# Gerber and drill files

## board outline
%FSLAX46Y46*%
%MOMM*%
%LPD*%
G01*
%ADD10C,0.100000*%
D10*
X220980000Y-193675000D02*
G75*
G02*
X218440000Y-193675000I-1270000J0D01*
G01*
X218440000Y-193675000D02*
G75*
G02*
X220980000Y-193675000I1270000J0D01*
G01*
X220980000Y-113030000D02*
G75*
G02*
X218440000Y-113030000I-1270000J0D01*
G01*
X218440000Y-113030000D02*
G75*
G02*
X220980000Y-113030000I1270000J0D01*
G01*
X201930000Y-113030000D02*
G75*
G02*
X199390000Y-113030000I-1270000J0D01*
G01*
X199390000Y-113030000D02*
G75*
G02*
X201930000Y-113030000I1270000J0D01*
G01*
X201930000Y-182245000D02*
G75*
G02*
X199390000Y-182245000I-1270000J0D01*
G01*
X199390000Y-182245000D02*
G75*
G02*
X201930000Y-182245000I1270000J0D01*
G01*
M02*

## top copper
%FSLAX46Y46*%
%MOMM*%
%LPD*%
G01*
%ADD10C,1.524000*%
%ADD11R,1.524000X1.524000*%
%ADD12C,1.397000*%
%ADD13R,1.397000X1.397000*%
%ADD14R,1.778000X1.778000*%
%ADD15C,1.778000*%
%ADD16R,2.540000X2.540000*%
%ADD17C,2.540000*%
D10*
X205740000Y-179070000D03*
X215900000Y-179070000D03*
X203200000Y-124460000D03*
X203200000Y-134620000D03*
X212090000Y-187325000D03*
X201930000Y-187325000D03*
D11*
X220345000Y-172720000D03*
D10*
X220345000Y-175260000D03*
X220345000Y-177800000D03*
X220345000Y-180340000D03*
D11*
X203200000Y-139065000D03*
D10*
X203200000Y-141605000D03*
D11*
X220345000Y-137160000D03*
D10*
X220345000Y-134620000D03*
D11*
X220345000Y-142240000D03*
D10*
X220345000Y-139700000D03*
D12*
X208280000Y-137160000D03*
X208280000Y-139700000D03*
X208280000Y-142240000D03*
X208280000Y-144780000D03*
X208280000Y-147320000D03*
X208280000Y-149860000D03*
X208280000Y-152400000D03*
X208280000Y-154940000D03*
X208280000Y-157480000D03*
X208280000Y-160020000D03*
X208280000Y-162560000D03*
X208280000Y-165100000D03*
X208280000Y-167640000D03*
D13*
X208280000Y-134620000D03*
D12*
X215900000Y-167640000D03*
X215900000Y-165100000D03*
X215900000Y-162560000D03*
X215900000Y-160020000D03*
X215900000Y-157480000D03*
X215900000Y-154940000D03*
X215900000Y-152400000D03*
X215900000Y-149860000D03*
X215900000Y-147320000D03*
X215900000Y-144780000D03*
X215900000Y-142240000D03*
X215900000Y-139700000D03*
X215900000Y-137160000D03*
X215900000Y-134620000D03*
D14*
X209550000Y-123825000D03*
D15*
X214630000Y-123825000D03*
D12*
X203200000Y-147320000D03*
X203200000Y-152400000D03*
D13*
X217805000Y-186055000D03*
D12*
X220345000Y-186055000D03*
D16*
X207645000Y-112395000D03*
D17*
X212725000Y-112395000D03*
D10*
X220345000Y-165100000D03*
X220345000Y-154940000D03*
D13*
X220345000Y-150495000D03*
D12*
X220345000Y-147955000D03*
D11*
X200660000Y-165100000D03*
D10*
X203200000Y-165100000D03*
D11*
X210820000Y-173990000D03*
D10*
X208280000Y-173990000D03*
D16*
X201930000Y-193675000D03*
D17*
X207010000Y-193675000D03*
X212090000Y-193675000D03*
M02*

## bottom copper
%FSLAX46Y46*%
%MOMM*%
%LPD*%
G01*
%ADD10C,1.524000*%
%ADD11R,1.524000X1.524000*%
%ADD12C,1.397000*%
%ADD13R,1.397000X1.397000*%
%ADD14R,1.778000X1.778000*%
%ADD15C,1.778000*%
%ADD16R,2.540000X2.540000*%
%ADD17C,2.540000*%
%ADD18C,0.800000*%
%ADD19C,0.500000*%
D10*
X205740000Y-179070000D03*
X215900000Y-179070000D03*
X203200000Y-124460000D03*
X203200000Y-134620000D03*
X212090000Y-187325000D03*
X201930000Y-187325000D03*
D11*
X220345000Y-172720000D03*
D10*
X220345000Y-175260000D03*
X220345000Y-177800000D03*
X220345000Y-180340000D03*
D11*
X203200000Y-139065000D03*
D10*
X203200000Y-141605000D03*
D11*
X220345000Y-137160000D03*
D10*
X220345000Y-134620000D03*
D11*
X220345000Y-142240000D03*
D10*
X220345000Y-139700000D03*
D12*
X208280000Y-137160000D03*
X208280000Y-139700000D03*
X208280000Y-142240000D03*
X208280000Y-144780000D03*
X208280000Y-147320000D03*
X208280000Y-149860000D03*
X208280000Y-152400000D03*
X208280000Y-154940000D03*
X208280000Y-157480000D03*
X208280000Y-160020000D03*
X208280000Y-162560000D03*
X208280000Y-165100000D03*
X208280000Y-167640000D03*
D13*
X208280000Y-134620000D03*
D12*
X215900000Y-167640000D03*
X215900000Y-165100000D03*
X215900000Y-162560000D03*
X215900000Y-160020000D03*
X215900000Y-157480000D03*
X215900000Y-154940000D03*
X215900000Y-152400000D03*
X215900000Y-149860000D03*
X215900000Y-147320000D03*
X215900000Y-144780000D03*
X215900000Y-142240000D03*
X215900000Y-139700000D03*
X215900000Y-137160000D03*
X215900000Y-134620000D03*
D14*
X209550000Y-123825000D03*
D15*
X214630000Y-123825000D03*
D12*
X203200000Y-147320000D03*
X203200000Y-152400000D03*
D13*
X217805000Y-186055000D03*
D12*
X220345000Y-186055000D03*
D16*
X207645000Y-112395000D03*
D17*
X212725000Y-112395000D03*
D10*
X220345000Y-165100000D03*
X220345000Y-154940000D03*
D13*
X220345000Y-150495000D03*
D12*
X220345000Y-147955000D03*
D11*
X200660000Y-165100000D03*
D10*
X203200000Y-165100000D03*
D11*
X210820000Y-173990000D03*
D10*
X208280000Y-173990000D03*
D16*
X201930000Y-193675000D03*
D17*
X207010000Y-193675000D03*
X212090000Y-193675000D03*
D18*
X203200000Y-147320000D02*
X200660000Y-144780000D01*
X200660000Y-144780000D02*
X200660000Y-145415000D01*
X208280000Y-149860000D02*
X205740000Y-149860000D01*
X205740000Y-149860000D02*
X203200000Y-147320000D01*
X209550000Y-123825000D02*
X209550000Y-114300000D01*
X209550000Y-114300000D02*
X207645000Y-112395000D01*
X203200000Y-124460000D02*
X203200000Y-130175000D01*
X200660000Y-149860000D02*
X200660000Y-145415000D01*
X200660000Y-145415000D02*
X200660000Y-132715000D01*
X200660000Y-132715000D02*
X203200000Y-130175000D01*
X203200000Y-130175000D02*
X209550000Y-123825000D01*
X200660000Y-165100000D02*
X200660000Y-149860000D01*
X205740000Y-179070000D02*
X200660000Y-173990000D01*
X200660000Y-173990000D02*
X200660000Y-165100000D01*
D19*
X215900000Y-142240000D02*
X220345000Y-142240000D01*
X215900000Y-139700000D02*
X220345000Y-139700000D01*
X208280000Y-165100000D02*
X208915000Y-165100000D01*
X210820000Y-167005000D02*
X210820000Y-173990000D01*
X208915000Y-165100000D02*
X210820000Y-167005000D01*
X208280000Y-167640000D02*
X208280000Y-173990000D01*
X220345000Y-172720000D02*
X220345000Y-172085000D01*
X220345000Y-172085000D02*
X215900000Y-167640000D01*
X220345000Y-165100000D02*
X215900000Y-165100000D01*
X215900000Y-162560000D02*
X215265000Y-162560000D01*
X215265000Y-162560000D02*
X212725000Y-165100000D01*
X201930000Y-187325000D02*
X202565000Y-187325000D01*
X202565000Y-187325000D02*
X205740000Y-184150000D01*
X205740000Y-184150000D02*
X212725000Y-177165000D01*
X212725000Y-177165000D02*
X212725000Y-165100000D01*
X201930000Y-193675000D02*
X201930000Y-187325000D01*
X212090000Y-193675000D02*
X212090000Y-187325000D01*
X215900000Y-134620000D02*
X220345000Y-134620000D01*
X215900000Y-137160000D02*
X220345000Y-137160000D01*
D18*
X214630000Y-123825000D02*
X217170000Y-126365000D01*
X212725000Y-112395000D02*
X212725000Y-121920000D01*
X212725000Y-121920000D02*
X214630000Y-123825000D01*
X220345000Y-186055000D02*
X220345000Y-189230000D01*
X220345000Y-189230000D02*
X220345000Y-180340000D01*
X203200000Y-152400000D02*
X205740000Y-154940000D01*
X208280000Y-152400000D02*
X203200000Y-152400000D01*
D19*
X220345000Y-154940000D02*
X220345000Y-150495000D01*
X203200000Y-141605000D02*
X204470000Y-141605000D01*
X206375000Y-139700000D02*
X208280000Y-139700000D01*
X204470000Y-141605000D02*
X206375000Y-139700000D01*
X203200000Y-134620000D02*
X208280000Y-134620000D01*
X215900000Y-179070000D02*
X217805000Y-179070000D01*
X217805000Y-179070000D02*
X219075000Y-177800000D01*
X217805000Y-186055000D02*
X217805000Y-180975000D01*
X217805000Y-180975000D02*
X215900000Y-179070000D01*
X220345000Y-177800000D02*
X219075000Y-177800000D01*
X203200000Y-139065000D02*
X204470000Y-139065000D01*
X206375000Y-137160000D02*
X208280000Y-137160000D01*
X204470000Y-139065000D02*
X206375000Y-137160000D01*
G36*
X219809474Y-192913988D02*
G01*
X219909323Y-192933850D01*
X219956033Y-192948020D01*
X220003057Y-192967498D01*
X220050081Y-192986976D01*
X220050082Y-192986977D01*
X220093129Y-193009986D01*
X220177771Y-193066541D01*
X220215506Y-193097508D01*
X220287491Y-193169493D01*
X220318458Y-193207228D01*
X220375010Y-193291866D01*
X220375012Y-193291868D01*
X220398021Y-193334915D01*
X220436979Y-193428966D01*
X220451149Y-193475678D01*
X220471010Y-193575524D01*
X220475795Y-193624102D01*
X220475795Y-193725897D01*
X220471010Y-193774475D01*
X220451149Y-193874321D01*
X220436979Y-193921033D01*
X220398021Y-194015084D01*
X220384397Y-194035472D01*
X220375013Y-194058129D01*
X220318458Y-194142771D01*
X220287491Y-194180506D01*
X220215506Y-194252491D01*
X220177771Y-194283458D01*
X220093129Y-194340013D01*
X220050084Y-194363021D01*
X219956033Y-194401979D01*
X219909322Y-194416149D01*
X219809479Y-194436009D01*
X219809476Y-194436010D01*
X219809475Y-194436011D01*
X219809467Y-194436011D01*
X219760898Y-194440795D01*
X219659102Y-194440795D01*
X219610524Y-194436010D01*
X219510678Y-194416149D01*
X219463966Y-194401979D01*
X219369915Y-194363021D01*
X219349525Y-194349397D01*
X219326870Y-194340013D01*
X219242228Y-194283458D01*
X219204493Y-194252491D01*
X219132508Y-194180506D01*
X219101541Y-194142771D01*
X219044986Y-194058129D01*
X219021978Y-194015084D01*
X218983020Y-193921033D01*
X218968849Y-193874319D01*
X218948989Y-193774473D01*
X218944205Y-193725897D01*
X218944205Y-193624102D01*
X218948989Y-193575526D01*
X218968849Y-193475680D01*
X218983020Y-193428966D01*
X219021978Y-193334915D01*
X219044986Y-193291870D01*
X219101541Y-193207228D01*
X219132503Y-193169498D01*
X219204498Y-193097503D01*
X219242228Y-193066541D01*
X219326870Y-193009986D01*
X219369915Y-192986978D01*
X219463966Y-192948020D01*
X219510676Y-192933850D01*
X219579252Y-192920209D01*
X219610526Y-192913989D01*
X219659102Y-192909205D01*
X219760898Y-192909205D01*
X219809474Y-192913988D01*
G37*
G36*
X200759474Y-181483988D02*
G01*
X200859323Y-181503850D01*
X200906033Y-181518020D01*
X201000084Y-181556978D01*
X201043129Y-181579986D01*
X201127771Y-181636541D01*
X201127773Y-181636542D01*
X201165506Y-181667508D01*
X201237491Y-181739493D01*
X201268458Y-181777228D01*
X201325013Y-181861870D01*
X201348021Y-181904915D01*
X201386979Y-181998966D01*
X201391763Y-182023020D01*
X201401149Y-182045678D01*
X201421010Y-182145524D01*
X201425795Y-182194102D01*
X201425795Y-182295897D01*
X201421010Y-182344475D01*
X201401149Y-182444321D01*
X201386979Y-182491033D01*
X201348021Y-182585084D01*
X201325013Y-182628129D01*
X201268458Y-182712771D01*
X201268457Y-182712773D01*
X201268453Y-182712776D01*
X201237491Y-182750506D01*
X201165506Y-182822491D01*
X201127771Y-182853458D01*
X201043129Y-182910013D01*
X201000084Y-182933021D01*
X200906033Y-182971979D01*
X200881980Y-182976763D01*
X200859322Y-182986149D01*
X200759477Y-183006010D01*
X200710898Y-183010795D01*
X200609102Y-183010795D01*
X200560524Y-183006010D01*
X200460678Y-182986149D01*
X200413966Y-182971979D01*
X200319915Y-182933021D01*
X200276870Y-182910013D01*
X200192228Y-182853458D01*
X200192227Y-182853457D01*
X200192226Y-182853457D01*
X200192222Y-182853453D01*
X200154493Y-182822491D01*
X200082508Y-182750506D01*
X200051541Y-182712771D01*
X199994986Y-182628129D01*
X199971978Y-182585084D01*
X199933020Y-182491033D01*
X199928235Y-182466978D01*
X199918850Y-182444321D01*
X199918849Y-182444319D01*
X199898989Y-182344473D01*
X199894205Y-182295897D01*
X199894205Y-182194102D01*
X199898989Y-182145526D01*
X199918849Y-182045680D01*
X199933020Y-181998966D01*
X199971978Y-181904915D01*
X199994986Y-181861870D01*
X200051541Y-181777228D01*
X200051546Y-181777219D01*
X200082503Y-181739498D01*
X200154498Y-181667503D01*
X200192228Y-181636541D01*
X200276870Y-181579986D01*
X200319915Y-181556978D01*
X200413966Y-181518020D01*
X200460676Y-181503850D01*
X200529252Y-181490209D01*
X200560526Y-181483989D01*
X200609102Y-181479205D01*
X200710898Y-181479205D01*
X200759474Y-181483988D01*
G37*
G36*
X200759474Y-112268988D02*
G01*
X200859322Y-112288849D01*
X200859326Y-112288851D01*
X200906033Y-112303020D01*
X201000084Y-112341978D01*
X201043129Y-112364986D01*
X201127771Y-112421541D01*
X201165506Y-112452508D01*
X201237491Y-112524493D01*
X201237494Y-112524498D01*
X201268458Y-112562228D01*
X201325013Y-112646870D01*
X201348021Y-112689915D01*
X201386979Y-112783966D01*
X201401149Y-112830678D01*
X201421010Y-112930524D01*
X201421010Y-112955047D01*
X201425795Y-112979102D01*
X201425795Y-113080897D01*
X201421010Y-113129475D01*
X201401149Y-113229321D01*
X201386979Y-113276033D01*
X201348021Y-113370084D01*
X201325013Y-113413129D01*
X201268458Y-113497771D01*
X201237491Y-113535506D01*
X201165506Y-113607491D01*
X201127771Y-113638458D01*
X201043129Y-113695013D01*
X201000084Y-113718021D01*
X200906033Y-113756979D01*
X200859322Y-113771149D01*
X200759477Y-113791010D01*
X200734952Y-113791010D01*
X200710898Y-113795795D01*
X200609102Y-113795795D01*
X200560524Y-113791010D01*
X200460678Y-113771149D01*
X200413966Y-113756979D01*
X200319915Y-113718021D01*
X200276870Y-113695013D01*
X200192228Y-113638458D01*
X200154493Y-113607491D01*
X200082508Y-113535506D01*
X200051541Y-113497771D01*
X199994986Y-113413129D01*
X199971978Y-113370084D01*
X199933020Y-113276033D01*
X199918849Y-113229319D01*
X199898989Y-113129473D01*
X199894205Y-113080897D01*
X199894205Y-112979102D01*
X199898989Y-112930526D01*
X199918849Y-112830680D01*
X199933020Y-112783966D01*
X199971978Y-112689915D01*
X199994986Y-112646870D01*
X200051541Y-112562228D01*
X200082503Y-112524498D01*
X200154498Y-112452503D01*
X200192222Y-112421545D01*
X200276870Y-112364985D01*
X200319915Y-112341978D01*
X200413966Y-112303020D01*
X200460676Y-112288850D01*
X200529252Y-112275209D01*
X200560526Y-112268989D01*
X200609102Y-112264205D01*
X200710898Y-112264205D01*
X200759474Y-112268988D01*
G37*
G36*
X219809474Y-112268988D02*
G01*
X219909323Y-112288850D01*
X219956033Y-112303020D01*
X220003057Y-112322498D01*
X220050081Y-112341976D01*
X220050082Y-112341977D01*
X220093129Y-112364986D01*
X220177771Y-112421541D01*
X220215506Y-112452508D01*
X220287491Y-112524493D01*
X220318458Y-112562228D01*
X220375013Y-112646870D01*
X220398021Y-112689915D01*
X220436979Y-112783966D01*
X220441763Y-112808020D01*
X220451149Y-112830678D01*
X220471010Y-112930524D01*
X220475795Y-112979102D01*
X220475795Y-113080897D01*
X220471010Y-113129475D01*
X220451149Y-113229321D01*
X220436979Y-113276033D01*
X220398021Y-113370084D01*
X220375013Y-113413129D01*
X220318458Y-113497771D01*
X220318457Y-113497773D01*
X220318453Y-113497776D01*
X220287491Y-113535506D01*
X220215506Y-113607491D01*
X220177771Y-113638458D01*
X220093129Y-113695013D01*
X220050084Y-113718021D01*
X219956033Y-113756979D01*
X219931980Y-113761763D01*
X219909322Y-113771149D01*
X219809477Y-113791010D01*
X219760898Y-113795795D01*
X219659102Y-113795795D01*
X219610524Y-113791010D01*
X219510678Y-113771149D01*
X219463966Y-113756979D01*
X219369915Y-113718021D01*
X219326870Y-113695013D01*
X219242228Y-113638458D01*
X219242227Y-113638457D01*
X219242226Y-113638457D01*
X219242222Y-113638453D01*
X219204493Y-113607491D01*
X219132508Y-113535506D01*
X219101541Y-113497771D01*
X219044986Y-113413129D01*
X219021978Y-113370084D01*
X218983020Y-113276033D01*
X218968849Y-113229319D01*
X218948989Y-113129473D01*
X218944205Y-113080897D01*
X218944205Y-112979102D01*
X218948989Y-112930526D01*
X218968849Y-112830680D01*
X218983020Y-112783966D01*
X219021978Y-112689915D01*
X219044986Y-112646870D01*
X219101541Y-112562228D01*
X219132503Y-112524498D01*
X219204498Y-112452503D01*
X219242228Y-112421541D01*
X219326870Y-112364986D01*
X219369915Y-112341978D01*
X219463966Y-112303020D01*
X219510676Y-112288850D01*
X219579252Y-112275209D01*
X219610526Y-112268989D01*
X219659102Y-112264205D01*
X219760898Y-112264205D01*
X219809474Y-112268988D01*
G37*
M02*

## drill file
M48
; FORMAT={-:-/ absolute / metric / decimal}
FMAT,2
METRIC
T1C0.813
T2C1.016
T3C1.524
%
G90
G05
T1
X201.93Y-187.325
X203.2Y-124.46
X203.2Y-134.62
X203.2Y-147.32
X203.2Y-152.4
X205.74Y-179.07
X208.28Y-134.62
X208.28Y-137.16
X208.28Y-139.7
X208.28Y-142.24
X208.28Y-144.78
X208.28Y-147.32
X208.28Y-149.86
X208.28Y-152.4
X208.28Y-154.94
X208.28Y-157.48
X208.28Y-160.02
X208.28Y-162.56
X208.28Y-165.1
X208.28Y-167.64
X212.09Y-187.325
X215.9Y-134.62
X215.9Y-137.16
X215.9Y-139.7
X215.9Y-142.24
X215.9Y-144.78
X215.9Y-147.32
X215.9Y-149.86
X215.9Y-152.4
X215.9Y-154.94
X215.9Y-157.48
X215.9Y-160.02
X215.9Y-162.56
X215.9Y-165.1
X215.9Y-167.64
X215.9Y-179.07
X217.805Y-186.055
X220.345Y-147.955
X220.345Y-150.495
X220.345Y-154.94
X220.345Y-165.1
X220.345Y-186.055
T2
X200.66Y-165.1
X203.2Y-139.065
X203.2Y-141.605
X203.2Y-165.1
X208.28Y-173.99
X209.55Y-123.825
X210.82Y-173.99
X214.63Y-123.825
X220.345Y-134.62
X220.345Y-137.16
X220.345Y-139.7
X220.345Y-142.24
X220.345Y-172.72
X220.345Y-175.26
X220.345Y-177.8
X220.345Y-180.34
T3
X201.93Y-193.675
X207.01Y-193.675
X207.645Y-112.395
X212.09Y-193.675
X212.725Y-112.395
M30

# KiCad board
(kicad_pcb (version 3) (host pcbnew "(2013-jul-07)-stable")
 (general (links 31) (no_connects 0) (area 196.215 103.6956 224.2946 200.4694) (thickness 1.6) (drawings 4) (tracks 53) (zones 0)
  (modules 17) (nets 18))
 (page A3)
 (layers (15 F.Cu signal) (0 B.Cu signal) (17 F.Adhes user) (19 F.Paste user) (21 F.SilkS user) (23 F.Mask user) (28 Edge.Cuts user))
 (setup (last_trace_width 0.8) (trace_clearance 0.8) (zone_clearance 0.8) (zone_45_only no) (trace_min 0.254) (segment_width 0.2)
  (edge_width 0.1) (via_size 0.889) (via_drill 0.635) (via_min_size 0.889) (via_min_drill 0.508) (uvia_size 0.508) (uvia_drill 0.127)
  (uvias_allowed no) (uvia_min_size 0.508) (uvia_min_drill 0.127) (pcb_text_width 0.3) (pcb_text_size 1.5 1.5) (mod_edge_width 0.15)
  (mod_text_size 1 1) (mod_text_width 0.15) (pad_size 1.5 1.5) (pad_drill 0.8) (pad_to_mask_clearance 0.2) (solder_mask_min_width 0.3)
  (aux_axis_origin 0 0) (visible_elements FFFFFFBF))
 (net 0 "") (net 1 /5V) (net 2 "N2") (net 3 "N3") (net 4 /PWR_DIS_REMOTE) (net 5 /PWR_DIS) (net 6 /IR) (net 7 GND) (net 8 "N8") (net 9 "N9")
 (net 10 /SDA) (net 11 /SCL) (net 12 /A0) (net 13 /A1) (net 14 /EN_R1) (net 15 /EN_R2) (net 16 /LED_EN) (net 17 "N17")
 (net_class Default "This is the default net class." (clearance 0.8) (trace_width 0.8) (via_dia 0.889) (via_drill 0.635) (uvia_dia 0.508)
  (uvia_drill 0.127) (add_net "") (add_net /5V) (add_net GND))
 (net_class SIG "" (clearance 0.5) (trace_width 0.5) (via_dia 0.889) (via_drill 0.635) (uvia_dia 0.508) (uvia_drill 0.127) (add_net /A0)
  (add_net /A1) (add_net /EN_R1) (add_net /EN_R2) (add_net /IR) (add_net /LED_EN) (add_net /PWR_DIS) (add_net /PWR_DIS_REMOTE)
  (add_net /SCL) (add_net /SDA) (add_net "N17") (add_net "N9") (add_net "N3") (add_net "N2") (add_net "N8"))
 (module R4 (layer F.Cu) (at 210.82 179.07) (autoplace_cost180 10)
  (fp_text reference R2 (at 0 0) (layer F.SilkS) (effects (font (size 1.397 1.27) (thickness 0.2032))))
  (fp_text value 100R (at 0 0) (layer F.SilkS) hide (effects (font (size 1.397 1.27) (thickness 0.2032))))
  (pad 1 thru_hole circle (at -5.08 0) (size 1.524 1.524) (drill 0.8128) (layers *.Cu *.Mask F.SilkS) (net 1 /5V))
  (pad 2 thru_hole circle (at 5.08 0) (size 1.524 1.524) (drill 0.8128) (layers *.Cu *.Mask F.SilkS) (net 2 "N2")))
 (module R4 (layer F.Cu) (at 203.2 129.54 270) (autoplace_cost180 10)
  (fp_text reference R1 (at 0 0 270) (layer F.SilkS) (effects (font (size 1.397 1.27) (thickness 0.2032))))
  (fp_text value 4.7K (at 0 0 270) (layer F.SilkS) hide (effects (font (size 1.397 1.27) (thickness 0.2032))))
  (pad 1 thru_hole circle (at -5.08 0 270) (size 1.524 1.524) (drill 0.8128) (layers *.Cu *.Mask F.SilkS) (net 1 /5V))
  (pad 2 thru_hole circle (at 5.08 0 270) (size 1.524 1.524) (drill 0.8128) (layers *.Cu *.Mask F.SilkS) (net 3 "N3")))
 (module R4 (layer F.Cu) (at 207.01 187.325 180) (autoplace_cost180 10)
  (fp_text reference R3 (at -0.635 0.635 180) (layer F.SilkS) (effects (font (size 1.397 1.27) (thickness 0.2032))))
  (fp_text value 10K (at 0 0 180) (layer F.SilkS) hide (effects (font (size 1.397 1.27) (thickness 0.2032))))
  (pad 1 thru_hole circle (at -5.08 0 180) (size 1.524 1.524) (drill 0.8128) (layers *.Cu *.Mask F.SilkS) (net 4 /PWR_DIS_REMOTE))
  (pad 2 thru_hole circle (at 5.08 0 180) (size 1.524 1.524) (drill 0.8128) (layers *.Cu *.Mask F.SilkS) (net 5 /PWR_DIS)))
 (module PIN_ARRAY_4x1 (layer F.Cu) (at 220.345 176.53 270)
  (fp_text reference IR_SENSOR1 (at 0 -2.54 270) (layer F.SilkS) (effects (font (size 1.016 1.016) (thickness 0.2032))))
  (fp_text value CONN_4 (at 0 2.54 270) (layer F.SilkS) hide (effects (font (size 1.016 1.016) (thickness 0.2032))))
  (pad 1 thru_hole rect (at -3.81 0 270) (size 1.524 1.524) (drill 1.016) (layers *.Cu *.Mask F.SilkS) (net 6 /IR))
  (pad 2 thru_hole circle (at -1.27 0 270) (size 1.524 1.524) (drill 1.016) (layers *.Cu *.Mask F.SilkS))
  (pad 3 thru_hole circle (at 1.27 0 270) (size 1.524 1.524) (drill 1.016) (layers *.Cu *.Mask F.SilkS) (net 2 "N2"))
  (pad 4 thru_hole circle (at 3.81 0 270) (size 1.524 1.524) (drill 1.016) (layers *.Cu *.Mask F.SilkS) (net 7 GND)))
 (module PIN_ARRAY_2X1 (layer F.Cu) (at 203.2 140.335 270)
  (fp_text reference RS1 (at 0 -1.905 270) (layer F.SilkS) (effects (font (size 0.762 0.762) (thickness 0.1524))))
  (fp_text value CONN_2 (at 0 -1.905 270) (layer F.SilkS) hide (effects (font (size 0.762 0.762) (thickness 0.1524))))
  (pad 1 thru_hole rect (at -1.27 0 270) (size 1.524 1.524) (drill 1.016) (layers *.Cu *.Mask F.SilkS) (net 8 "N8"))
  (pad 2 thru_hole circle (at 1.27 0 270) (size 1.524 1.524) (drill 1.016) (layers *.Cu *.Mask F.SilkS) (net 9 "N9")))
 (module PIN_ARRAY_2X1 (layer F.Cu) (at 220.345 135.89 90)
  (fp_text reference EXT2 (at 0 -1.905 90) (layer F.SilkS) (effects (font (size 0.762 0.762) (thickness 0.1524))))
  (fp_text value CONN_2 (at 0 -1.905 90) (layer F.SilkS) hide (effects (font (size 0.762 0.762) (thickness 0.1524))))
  (pad 1 thru_hole rect (at -1.27 0 90) (size 1.524 1.524) (drill 1.016) (layers *.Cu *.Mask F.SilkS) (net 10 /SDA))
  (pad 2 thru_hole circle (at 1.27 0 90) (size 1.524 1.524) (drill 1.016) (layers *.Cu *.Mask F.SilkS) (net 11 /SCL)))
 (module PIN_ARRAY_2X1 (layer F.Cu) (at 220.345 140.97 90)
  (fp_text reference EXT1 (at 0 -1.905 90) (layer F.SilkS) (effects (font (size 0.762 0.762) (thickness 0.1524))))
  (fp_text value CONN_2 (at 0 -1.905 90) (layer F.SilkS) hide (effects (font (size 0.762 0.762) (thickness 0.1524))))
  (pad 1 thru_hole rect (at -1.27 0 90) (size 1.524 1.524) (drill 1.016) (layers *.Cu *.Mask F.SilkS) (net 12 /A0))
  (pad 2 thru_hole circle (at 1.27 0 90) (size 1.524 1.524) (drill 1.016) (layers *.Cu *.Mask F.SilkS) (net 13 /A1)))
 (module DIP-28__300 (layer F.Cu) (at 212.09 151.13 270)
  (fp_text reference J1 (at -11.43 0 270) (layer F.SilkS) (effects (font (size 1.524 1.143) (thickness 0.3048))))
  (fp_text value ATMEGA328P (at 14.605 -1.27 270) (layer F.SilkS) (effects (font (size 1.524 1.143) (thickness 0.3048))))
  (pad 2 thru_hole circle (at -13.97 3.81 270) (size 1.397 1.397) (drill 0.8128) (layers *.Cu *.Mask F.SilkS) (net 8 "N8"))
  (pad 3 thru_hole circle (at -11.43 3.81 270) (size 1.397 1.397) (drill 0.8128) (layers *.Cu *.Mask F.SilkS) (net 9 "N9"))
  (pad 4 thru_hole circle (at -8.89 3.81 270) (size 1.397 1.397) (drill 0.8128) (layers *.Cu *.Mask F.SilkS))
  (pad 5 thru_hole circle (at -6.35 3.81 270) (size 1.397 1.397) (drill 0.8128) (layers *.Cu *.Mask F.SilkS))
  (pad 6 thru_hole circle (at -3.81 3.81 270) (size 1.397 1.397) (drill 0.8128) (layers *.Cu *.Mask F.SilkS))
  (pad 7 thru_hole circle (at -1.27 3.81 270) (size 1.397 1.397) (drill 0.8128) (layers *.Cu *.Mask F.SilkS) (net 1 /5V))
  (pad 8 thru_hole circle (at 1.27 3.81 270) (size 1.397 1.397) (drill 0.8128) (layers *.Cu *.Mask F.SilkS) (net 7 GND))
  (pad 9 thru_hole circle (at 3.81 3.81 270) (size 1.397 1.397) (drill 0.8128) (layers *.Cu *.Mask F.SilkS))
  (pad 10 thru_hole circle (at 6.35 3.81 270) (size 1.397 1.397) (drill 0.8128) (layers *.Cu *.Mask F.SilkS))
  (pad 11 thru_hole circle (at 8.89 3.81 270) (size 1.397 1.397) (drill 0.8128) (layers *.Cu *.Mask F.SilkS))
  (pad 12 thru_hole circle (at 11.43 3.81 270) (size 1.397 1.397) (drill 0.8128) (layers *.Cu *.Mask F.SilkS))
  (pad 13 thru_hole circle (at 13.97 3.81 270) (size 1.397 1.397) (drill 0.8128) (layers *.Cu *.Mask F.SilkS) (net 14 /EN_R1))
  (pad 14 thru_hole circle (at 16.51 3.81 270) (size 1.397 1.397) (drill 0.8128) (layers *.Cu *.Mask F.SilkS) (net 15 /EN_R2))
  (pad 1 thru_hole rect (at -16.51 3.81 270) (size 1.397 1.397) (drill 0.8128) (layers *.Cu *.Mask F.SilkS) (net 3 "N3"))
  (pad 15 thru_hole circle (at 16.51 -3.81 270) (size 1.397 1.397) (drill 0.8128) (layers *.Cu *.Mask F.SilkS) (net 6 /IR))
  (pad 16 thru_hole circle (at 13.97 -3.81 270) (size 1.397 1.397) (drill 0.8128) (layers *.Cu *.Mask F.SilkS) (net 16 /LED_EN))
  (pad 17 thru_hole circle (at 11.43 -3.81 270) (size 1.397 1.397) (drill 0.8128) (layers *.Cu *.Mask F.SilkS) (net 5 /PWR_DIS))
  (pad 18 thru_hole circle (at 8.89 -3.81 270) (size 1.397 1.397) (drill 0.8128) (layers *.Cu *.Mask F.SilkS))
  (pad 19 thru_hole circle (at 6.35 -3.81 270) (size 1.397 1.397) (drill 0.8128) (layers *.Cu *.Mask F.SilkS))
  (pad 20 thru_hole circle (at 3.81 -3.81 270) (size 1.397 1.397) (drill 0.8128) (layers *.Cu *.Mask F.SilkS))
  (pad 21 thru_hole circle (at 1.27 -3.81 270) (size 1.397 1.397) (drill 0.8128) (layers *.Cu *.Mask F.SilkS))
  (pad 22 thru_hole circle (at -1.27 -3.81 270) (size 1.397 1.397) (drill 0.8128) (layers *.Cu *.Mask F.SilkS))
  (pad 23 thru_hole circle (at -3.81 -3.81 270) (size 1.397 1.397) (drill 0.8128) (layers *.Cu *.Mask F.SilkS))
  (pad 24 thru_hole circle (at -6.35 -3.81 270) (size 1.397 1.397) (drill 0.8128) (layers *.Cu *.Mask F.SilkS))
  (pad 25 thru_hole circle (at -8.89 -3.81 270) (size 1.397 1.397) (drill 0.8128) (layers *.Cu *.Mask F.SilkS) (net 12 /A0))
  (pad 26 thru_hole circle (at -11.43 -3.81 270) (size 1.397 1.397) (drill 0.8128) (layers *.Cu *.Mask F.SilkS) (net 13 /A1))
  (pad 27 thru_hole circle (at -13.97 -3.81 270) (size 1.397 1.397) (drill 0.8128) (layers *.Cu *.Mask F.SilkS) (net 10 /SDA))
  (pad 28 thru_hole circle (at -16.51 -3.81 270) (size 1.397 1.397) (drill 0.8128) (layers *.Cu *.Mask F.SilkS) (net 11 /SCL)))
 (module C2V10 (layer F.Cu) (at 212.09 123.825)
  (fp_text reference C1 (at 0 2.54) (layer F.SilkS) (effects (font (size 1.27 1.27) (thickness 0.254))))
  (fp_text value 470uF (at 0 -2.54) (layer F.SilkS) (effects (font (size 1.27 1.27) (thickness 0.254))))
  (pad 1 thru_hole rect (at -2.54 0) (size 1.778 1.778) (drill 1.016) (layers *.Cu *.Mask F.SilkS) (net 1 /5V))
  (pad 2 thru_hole circle (at 2.54 0) (size 1.778 1.778) (drill 1.016) (layers *.Cu *.Mask F.SilkS) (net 7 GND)))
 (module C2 (layer F.Cu) (at 203.2 149.86 270)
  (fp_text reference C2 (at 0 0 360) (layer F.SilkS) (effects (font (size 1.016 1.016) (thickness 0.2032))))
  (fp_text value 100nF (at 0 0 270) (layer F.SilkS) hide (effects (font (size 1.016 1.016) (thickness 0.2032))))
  (pad 1 thru_hole circle (at -2.54 0 270) (size 1.397 1.397) (drill 0.8128) (layers *.Cu *.Mask F.SilkS) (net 1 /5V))
  (pad 2 thru_hole circle (at 2.54 0 270) (size 1.397 1.397) (drill 0.8128) (layers *.Cu *.Mask F.SilkS) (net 7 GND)))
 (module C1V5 (layer F.Cu) (at 219.075 186.055)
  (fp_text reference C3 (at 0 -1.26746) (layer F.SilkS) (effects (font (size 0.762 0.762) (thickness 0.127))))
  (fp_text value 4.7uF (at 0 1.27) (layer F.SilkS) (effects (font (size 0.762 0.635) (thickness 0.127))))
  (pad 1 thru_hole rect (at -1.27 0) (size 1.397 1.397) (drill 0.8128) (layers *.Cu *.Mask F.SilkS) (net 2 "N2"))
  (pad 2 thru_hole circle (at 1.27 0) (size 1.397 1.397) (drill 0.8128) (layers *.Cu *.Mask F.SilkS) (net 7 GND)))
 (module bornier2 (layer F.Cu) (at 210.185 112.395)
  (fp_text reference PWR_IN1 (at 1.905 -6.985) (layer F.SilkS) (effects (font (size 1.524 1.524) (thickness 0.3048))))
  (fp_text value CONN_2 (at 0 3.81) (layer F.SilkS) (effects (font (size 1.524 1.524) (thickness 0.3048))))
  (pad 1 thru_hole rect (at -2.54 0) (size 2.54 2.54) (drill 1.524) (layers *.Cu *.Mask F.SilkS) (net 1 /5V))
  (pad 2 thru_hole circle (at 2.54 0) (size 2.54 2.54) (drill 1.524) (layers *.Cu *.Mask F.SilkS) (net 7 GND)))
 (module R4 (layer F.Cu) (at 220.345 160.02 90) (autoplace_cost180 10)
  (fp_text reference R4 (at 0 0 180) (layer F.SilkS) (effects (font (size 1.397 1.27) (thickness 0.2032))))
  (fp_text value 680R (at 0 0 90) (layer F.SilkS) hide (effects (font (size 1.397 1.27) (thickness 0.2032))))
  (pad 1 thru_hole circle (at -5.08 0 90) (size 1.524 1.524) (drill 0.8128) (layers *.Cu *.Mask F.SilkS) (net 16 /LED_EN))
  (pad 2 thru_hole circle (at 5.08 0 90) (size 1.524 1.524) (drill 0.8128) (layers *.Cu *.Mask F.SilkS) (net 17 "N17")))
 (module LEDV (layer F.Cu) (at 220.345 149.225 90)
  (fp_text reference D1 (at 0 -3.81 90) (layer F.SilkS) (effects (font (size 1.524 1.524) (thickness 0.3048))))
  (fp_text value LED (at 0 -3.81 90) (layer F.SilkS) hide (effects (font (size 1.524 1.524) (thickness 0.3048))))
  (pad 1 thru_hole rect (at -1.27 0 90) (size 1.397 1.397) (drill 0.8128) (layers *.Cu *.Mask F.SilkS) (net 17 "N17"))
  (pad 2 thru_hole circle (at 1.27 0 90) (size 1.397 1.397) (drill 0.8128) (layers *.Cu *.Mask F.SilkS) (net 7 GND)))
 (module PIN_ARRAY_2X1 (layer F.Cu) (at 201.93 165.1)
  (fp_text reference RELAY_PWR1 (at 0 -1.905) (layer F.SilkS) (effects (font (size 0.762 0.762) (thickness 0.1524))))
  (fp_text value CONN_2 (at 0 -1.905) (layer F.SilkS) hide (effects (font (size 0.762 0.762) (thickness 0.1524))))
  (pad 1 thru_hole rect (at -1.27 0) (size 1.524 1.524) (drill 1.016) (layers *.Cu *.Mask F.SilkS) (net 1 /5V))
  (pad 2 thru_hole circle (at 1.27 0) (size 1.524 1.524) (drill 1.016) (layers *.Cu *.Mask F.SilkS) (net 7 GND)))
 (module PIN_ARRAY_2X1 (layer F.Cu) (at 209.55 173.99 180)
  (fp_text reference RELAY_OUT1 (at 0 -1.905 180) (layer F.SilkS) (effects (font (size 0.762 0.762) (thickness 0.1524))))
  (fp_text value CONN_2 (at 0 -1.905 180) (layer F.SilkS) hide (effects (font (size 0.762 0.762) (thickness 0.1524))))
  (pad 1 thru_hole rect (at -1.27 0 180) (size 1.524 1.524) (drill 1.016) (layers *.Cu *.Mask F.SilkS) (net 14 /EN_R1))
  (pad 2 thru_hole circle (at 1.27 0 180) (size 1.524 1.524) (drill 1.016) (layers *.Cu *.Mask F.SilkS) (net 15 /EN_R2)))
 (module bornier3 (layer F.Cu) (at 207.01 193.675)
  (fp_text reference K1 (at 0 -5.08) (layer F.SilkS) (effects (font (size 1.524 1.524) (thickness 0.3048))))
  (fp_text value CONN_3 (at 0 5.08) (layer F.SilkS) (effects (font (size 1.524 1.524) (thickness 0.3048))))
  (pad 1 thru_hole rect (at -5.08 0) (size 2.54 2.54) (drill 1.524) (layers *.Cu *.Mask F.SilkS) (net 5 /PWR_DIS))
  (pad 2 thru_hole circle (at 0 0) (size 2.54 2.54) (drill 1.524) (layers *.Cu *.Mask F.SilkS) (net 7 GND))
  (pad 3 thru_hole circle (at 5.08 0) (size 2.54 2.54) (drill 1.524) (layers *.Cu *.Mask F.SilkS) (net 4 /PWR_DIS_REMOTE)))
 (gr_circle (center 219.71 193.675) (end 218.44 193.675) (layer Edge.Cuts) (width 0.1))
 (gr_circle (center 219.71 113.03) (end 220.98 113.03) (layer Edge.Cuts) (width 0.1))
 (gr_circle (center 200.66 113.03) (end 201.93 113.03) (layer Edge.Cuts) (width 0.1))
 (gr_circle (center 200.66 182.245) (end 201.93 182.245) (layer Edge.Cuts) (width 0.1))
 (segment (start 203.2 147.32) (end 200.66 144.78) (width 0.8) (layer B.Cu) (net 1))
 (segment (start 200.66 144.78) (end 200.66 145.415) (width 0.8) (layer B.Cu) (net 1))
 (segment (start 208.28 149.86) (end 205.74 149.86) (width 0.8) (layer B.Cu) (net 1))
 (segment (start 205.74 149.86) (end 203.2 147.32) (width 0.8) (layer B.Cu) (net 1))
 (segment (start 209.55 123.825) (end 209.55 114.3) (width 0.8) (layer B.Cu) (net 1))
 (segment (start 209.55 114.3) (end 207.645 112.395) (width 0.8) (layer B.Cu) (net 1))
 (segment (start 203.2 124.46) (end 203.2 130.175) (width 0.8) (layer B.Cu) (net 1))
 (segment (start 200.66 149.86) (end 200.66 145.415) (width 0.8) (layer B.Cu) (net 1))
 (segment (start 200.66 145.415) (end 200.66 132.715) (width 0.8) (layer B.Cu) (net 1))
 (segment (start 200.66 132.715) (end 203.2 130.175) (width 0.8) (layer B.Cu) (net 1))
 (segment (start 203.2 130.175) (end 209.55 123.825) (width 0.8) (layer B.Cu) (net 1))
 (segment (start 200.66 165.1) (end 200.66 149.86) (width 0.8) (layer B.Cu) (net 1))
 (segment (start 205.74 179.07) (end 200.66 173.99) (width 0.8) (layer B.Cu) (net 1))
 (segment (start 200.66 173.99) (end 200.66 165.1) (width 0.8) (layer B.Cu) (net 1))
 (segment (start 215.9 142.24) (end 220.345 142.24) (width 0.5) (layer B.Cu) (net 12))
 (segment (start 215.9 139.7) (end 220.345 139.7) (width 0.5) (layer B.Cu) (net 13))
 (segment (start 208.28 165.1) (end 208.915 165.1) (width 0.5) (layer B.Cu) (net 14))
 (segment (start 210.82 167.005) (end 210.82 173.99) (width 0.5) (layer B.Cu) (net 14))
 (segment (start 208.915 165.1) (end 210.82 167.005) (width 0.5) (layer B.Cu) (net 14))
 (segment (start 208.28 167.64) (end 208.28 173.99) (width 0.5) (layer B.Cu) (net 15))
 (segment (start 220.345 172.72) (end 220.345 172.085) (width 0.5) (layer B.Cu) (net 6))
 (segment (start 220.345 172.085) (end 215.9 167.64) (width 0.5) (layer B.Cu) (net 6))
 (segment (start 220.345 165.1) (end 215.9 165.1) (width 0.5) (layer B.Cu) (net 16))
 (segment (start 215.9 162.56) (end 215.265 162.56) (width 0.5) (layer B.Cu) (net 5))
 (segment (start 215.265 162.56) (end 212.725 165.1) (width 0.5) (layer B.Cu) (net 5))
 (segment (start 201.93 187.325) (end 202.565 187.325) (width 0.5) (layer B.Cu) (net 5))
 (segment (start 202.565 187.325) (end 205.74 184.15) (width 0.5) (layer B.Cu) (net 5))
 (segment (start 205.74 184.15) (end 212.725 177.165) (width 0.5) (layer B.Cu) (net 5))
 (segment (start 212.725 177.165) (end 212.725 165.1) (width 0.5) (layer B.Cu) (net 5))
 (segment (start 201.93 193.675) (end 201.93 187.325) (width 0.5) (layer B.Cu) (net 5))
 (segment (start 212.09 193.675) (end 212.09 187.325) (width 0.5) (layer B.Cu) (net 4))
 (segment (start 215.9 134.62) (end 220.345 134.62) (width 0.5) (layer B.Cu) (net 11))
 (segment (start 215.9 137.16) (end 220.345 137.16) (width 0.5) (layer B.Cu) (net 10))
 (segment (start 214.63 123.825) (end 217.17 126.365) (width 0.8) (layer B.Cu) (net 7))
 (segment (start 212.725 112.395) (end 212.725 121.92) (width 0.8) (layer B.Cu) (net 7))
 (segment (start 212.725 121.92) (end 214.63 123.825) (width 0.8) (layer B.Cu) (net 7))
 (segment (start 220.345 186.055) (end 220.345 189.23) (width 0.8) (layer B.Cu) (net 7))
 (segment (start 220.345 189.23) (end 220.345 180.34) (width 0.8) (layer B.Cu) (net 7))
 (segment (start 203.2 152.4) (end 205.74 154.94) (width 0.8) (layer B.Cu) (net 7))
 (segment (start 208.28 152.4) (end 203.2 152.4) (width 0.8) (layer B.Cu) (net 7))
 (segment (start 220.345 154.94) (end 220.345 150.495) (width 0.5) (layer B.Cu) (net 17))
 (segment (start 203.2 141.605) (end 204.47 141.605) (width 0.5) (layer B.Cu) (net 9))
 (segment (start 206.375 139.7) (end 208.28 139.7) (width 0.5) (layer B.Cu) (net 9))
 (segment (start 204.47 141.605) (end 206.375 139.7) (width 0.5) (layer B.Cu) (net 9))
 (segment (start 203.2 134.62) (end 208.28 134.62) (width 0.5) (layer B.Cu) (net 3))
 (segment (start 215.9 179.07) (end 217.805 179.07) (width 0.5) (layer B.Cu) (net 2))
 (segment (start 217.805 179.07) (end 219.075 177.8) (width 0.5) (layer B.Cu) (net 2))
 (segment (start 217.805 186.055) (end 217.805 180.975) (width 0.5) (layer B.Cu) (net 2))
 (segment (start 217.805 180.975) (end 215.9 179.07) (width 0.5) (layer B.Cu) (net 2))
 (segment (start 220.345 177.8) (end 219.075 177.8) (width 0.5) (layer B.Cu) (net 2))
 (segment (start 203.2 139.065) (end 204.47 139.065) (width 0.5) (layer B.Cu) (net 8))
 (segment (start 206.375 137.16) (end 208.28 137.16) (width 0.5) (layer B.Cu) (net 8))
 (segment (start 204.47 139.065) (end 206.375 137.16) (width 0.5) (layer B.Cu) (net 8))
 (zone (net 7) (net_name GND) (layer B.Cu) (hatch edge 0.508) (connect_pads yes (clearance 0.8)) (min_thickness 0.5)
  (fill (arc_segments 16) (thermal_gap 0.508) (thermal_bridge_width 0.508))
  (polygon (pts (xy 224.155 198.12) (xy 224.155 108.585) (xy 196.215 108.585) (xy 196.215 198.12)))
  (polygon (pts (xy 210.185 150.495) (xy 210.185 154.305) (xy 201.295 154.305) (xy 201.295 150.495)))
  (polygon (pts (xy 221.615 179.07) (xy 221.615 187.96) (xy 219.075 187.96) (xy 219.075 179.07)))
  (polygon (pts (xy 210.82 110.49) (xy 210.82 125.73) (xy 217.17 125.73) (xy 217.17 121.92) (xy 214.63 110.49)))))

